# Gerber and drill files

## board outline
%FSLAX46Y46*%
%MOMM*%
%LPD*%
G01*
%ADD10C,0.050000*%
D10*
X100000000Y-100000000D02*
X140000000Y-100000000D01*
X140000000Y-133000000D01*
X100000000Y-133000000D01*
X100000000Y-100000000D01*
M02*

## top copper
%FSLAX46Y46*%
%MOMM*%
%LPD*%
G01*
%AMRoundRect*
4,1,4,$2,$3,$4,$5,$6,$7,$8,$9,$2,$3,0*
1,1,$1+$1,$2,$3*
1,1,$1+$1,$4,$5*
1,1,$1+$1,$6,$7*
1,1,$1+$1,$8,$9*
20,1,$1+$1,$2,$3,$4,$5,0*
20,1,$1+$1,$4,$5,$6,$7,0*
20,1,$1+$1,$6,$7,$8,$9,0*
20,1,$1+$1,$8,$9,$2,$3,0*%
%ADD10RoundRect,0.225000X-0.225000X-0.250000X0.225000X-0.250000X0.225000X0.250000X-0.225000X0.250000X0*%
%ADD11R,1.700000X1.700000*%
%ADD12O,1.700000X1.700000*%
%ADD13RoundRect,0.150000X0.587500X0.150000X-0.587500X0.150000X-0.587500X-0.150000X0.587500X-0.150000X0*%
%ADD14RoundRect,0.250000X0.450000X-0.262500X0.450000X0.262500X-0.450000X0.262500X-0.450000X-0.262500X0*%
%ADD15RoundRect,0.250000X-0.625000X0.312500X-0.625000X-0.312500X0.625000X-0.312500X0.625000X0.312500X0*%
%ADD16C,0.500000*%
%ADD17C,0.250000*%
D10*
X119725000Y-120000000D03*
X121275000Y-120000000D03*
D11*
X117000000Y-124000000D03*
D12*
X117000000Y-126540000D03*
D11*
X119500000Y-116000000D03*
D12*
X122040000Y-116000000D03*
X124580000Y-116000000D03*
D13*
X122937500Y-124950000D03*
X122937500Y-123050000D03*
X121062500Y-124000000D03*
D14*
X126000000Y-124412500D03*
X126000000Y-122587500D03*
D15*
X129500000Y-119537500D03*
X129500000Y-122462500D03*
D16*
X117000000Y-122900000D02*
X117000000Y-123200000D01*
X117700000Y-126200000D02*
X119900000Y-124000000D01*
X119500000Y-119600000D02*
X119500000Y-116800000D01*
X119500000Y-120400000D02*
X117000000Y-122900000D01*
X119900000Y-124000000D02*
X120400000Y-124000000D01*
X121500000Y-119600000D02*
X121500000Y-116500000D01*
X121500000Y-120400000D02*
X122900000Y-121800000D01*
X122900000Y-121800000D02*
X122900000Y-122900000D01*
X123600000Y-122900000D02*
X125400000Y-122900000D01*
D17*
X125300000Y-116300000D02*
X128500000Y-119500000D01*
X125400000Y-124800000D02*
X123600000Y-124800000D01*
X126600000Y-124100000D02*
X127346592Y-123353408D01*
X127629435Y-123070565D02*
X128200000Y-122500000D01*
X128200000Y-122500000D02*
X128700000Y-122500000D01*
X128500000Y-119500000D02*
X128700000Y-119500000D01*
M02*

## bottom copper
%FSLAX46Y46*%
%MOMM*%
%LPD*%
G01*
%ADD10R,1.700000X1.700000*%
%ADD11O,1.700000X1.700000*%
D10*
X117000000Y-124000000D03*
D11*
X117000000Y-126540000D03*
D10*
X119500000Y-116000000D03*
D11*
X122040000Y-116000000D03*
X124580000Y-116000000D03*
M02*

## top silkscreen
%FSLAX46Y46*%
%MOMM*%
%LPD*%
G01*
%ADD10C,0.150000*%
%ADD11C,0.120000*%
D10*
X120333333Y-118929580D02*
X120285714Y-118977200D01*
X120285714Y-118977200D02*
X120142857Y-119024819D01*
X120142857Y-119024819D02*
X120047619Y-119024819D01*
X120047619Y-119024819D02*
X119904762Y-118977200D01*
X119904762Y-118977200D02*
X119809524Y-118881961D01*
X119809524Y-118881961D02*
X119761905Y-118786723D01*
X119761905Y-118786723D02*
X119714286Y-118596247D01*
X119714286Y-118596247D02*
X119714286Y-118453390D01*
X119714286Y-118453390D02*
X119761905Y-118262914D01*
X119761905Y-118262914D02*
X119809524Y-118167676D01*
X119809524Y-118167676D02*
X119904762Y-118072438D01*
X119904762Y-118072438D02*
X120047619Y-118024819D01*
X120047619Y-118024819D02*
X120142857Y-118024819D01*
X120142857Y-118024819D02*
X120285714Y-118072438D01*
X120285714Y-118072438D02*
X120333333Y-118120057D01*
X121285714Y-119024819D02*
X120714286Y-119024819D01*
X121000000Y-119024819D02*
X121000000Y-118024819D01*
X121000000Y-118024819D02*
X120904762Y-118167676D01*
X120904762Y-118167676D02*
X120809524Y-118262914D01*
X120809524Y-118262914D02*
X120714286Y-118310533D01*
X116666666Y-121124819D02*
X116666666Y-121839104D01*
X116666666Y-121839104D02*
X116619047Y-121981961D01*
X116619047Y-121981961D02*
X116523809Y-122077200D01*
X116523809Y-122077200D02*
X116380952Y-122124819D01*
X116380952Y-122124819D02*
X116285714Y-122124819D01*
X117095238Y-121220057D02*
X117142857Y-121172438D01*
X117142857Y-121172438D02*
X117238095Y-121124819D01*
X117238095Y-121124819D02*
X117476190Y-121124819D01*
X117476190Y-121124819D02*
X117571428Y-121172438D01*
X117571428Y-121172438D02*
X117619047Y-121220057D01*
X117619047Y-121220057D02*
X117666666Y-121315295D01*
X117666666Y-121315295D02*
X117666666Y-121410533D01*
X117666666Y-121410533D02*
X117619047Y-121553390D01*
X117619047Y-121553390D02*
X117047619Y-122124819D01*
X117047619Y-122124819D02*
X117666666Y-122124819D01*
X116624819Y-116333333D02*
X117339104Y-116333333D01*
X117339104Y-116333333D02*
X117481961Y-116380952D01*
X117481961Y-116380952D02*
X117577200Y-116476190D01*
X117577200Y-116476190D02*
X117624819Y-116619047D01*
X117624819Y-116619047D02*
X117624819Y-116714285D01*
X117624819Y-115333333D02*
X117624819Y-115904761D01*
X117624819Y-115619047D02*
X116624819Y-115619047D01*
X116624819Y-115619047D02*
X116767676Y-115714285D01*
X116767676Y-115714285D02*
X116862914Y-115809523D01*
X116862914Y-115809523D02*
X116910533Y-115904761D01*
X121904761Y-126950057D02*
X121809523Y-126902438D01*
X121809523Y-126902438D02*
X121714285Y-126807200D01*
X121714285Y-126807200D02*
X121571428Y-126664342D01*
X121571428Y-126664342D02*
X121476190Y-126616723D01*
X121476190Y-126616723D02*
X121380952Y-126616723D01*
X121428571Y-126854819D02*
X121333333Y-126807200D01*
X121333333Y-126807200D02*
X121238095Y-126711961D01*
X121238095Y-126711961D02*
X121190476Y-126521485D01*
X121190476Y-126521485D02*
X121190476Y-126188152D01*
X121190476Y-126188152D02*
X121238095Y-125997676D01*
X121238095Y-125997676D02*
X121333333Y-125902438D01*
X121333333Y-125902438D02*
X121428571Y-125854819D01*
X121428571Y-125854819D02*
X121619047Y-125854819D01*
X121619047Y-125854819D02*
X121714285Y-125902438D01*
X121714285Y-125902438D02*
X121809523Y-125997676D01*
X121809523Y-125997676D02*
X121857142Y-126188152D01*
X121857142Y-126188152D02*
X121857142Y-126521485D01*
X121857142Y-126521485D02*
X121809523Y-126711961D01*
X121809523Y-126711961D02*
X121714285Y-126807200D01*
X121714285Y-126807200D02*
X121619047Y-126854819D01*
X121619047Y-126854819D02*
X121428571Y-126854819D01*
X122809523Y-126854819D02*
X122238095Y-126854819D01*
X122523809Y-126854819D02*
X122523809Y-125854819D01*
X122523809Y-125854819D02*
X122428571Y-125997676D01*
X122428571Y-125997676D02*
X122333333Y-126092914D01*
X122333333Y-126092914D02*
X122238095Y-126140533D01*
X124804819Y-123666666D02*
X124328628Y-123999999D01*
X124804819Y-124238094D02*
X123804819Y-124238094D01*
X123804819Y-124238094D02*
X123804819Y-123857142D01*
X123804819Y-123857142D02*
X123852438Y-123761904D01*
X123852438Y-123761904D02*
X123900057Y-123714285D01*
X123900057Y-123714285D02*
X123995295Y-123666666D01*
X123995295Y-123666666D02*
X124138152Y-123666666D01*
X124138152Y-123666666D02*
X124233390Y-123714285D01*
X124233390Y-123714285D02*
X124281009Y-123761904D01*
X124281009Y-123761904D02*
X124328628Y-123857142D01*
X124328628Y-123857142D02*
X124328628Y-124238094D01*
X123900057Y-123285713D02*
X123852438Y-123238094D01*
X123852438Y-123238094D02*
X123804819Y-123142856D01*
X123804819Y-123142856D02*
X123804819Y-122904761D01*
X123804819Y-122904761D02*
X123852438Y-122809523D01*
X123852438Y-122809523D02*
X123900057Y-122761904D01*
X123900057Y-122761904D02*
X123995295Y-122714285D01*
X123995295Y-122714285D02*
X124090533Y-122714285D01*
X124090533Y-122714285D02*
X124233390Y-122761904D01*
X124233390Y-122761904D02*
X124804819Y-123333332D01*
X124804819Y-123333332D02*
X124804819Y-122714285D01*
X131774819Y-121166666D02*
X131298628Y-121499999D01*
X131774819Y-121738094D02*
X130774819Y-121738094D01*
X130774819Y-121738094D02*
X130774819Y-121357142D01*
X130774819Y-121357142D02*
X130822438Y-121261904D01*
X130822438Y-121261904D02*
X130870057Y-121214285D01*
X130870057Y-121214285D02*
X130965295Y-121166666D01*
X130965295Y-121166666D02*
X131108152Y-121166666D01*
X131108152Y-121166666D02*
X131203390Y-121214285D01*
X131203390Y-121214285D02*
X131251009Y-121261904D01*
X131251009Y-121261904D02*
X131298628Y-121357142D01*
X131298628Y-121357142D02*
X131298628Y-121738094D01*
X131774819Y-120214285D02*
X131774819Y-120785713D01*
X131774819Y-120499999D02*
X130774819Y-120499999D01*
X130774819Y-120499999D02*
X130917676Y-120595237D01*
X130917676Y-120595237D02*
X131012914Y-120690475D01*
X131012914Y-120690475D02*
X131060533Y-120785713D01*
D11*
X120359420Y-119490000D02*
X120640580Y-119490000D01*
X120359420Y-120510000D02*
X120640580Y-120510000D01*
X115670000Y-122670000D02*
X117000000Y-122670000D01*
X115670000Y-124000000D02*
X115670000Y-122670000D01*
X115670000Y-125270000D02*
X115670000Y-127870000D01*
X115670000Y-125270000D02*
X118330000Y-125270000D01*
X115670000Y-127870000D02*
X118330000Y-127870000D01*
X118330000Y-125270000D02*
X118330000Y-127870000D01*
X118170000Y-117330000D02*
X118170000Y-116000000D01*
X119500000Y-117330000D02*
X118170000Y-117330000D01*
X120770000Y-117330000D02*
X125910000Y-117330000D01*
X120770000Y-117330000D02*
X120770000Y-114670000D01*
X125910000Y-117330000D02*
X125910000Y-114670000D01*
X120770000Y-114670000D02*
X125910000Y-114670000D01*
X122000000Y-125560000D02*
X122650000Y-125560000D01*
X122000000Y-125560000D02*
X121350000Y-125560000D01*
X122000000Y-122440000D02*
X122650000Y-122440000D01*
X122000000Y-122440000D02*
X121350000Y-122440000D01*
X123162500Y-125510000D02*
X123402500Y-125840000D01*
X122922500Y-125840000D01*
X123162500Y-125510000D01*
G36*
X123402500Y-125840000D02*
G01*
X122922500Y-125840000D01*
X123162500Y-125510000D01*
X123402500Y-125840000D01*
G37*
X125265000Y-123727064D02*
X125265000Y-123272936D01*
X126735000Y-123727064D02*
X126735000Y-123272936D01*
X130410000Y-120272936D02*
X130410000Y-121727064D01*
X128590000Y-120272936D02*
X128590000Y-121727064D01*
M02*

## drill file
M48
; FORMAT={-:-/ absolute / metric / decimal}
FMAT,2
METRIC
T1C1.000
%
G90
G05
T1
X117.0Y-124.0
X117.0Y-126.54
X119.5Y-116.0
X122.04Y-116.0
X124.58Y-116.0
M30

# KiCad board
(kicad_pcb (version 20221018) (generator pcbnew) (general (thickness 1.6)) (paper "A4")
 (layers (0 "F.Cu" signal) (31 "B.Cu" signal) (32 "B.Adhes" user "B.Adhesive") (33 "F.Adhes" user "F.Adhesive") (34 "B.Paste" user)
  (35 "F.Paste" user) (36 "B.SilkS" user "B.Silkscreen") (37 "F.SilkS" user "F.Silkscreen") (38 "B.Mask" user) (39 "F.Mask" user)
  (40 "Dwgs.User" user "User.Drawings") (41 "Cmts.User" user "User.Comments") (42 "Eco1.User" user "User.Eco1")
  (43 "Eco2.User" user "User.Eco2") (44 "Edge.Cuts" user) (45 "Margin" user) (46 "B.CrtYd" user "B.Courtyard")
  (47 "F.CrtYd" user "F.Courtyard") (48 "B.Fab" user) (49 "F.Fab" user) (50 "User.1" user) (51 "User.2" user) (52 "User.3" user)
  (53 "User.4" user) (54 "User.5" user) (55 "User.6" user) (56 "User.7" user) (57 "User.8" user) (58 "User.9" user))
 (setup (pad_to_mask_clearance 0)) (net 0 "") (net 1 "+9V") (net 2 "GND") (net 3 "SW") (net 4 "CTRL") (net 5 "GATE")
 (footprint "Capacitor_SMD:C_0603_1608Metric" (layer "F.Cu") (at 120.5 120)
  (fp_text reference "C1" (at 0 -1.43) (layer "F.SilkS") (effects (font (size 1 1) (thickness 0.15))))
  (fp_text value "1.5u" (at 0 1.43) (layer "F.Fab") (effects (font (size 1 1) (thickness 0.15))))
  (fp_line (start -0.14058 -0.51) (end 0.14058 -0.51) (stroke (width 0.12) (type solid)) (layer "F.SilkS"))
  (fp_line (start -0.14058 0.51) (end 0.14058 0.51) (stroke (width 0.12) (type solid)) (layer "F.SilkS"))
  (pad "1" smd roundrect (at -0.775 0) (size 0.9 0.95) (layers "F.Cu" "F.Paste" "F.Mask") (roundrect_rratio 0.25) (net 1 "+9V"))
  (pad "2" smd roundrect (at 0.775 0) (size 0.9 0.95) (layers "F.Cu" "F.Paste" "F.Mask") (roundrect_rratio 0.25) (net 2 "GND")))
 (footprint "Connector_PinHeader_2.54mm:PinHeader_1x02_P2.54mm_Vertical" (layer "F.Cu") (at 117 124)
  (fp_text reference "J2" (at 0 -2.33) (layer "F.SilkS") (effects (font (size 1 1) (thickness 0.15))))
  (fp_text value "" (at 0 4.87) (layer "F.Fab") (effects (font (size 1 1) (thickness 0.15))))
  (fp_line (start -1.33 -1.33) (end 0 -1.33) (stroke (width 0.12) (type solid)) (layer "F.SilkS"))
  (fp_line (start -1.33 0) (end -1.33 -1.33) (stroke (width 0.12) (type solid)) (layer "F.SilkS"))
  (fp_line (start -1.33 1.27) (end -1.33 3.87) (stroke (width 0.12) (type solid)) (layer "F.SilkS"))
  (fp_line (start -1.33 1.27) (end 1.33 1.27) (stroke (width 0.12) (type solid)) (layer "F.SilkS"))
  (fp_line (start -1.33 3.87) (end 1.33 3.87) (stroke (width 0.12) (type solid)) (layer "F.SilkS"))
  (fp_line (start 1.33 1.27) (end 1.33 3.87) (stroke (width 0.12) (type solid)) (layer "F.SilkS"))
  (pad "1" thru_hole rect (at 0 0) (size 1.7 1.7) (drill 1) (layers "*.Cu" "*.Mask") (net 1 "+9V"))
  (pad "2" thru_hole oval (at 0 2.54) (size 1.7 1.7) (drill 1) (layers "*.Cu" "*.Mask") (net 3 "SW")))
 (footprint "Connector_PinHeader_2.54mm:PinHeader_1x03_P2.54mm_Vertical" (layer "F.Cu") (at 119.5 116 90)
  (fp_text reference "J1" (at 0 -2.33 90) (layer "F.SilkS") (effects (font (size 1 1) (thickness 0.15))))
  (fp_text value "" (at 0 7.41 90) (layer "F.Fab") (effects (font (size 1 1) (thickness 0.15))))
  (fp_line (start -1.33 -1.33) (end 0 -1.33) (stroke (width 0.12) (type solid)) (layer "F.SilkS"))
  (fp_line (start -1.33 0) (end -1.33 -1.33) (stroke (width 0.12) (type solid)) (layer "F.SilkS"))
  (fp_line (start -1.33 1.27) (end -1.33 6.41) (stroke (width 0.12) (type solid)) (layer "F.SilkS"))
  (fp_line (start -1.33 1.27) (end 1.33 1.27) (stroke (width 0.12) (type solid)) (layer "F.SilkS"))
  (fp_line (start -1.33 6.41) (end 1.33 6.41) (stroke (width 0.12) (type solid)) (layer "F.SilkS"))
  (fp_line (start 1.33 1.27) (end 1.33 6.41) (stroke (width 0.12) (type solid)) (layer "F.SilkS"))
  (pad "1" thru_hole rect (at 0 0 90) (size 1.7 1.7) (drill 1) (layers "*.Cu" "*.Mask") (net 1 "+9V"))
  (pad "2" thru_hole oval (at 0 2.54 90) (size 1.7 1.7) (drill 1) (layers "*.Cu" "*.Mask") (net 2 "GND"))
  (pad "3" thru_hole oval (at 0 5.08 90) (size 1.7 1.7) (drill 1) (layers "*.Cu" "*.Mask") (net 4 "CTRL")))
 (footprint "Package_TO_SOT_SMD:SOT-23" (layer "F.Cu") (at 122 124 180)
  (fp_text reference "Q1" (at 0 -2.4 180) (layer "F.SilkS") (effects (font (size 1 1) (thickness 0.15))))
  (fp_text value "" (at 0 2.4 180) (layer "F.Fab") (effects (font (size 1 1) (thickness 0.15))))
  (fp_line (start 0 -1.56) (end -0.65 -1.56) (stroke (width 0.12) (type solid)) (layer "F.SilkS"))
  (fp_line (start 0 -1.56) (end 0.65 -1.56) (stroke (width 0.12) (type solid)) (layer "F.SilkS"))
  (fp_line (start 0 1.56) (end -0.65 1.56) (stroke (width 0.12) (type solid)) (layer "F.SilkS"))
  (fp_line (start 0 1.56) (end 0.65 1.56) (stroke (width 0.12) (type solid)) (layer "F.SilkS"))
  (fp_poly
   (pts (xy -1.1625 -1.51) (xy -1.4025 -1.84) (xy -0.9225 -1.84) (xy -1.1625 -1.51)) (stroke (width 0.12) (type solid)) (fill solid)
   (layer "F.SilkS"))
  (pad "1" smd roundrect (at -0.9375 -0.95 180) (size 1.475 0.6) (layers "F.Cu" "F.Paste" "F.Mask") (roundrect_rratio 0.25) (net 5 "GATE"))
  (pad "2" smd roundrect (at -0.9375 0.95 180) (size 1.475 0.6) (layers "F.Cu" "F.Paste" "F.Mask") (roundrect_rratio 0.25) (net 2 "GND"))
  (pad "3" smd roundrect (at 0.9375 0 180) (size 1.475 0.6) (layers "F.Cu" "F.Paste" "F.Mask") (roundrect_rratio 0.25) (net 3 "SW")))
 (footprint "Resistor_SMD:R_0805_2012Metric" (layer "F.Cu") (at 126 123.5 90)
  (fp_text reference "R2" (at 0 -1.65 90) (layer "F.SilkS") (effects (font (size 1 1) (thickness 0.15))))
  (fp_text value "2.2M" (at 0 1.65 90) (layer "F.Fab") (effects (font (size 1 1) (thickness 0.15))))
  (fp_line (start -0.227064 -0.735) (end 0.227064 -0.735) (stroke (width 0.12) (type solid)) (layer "F.SilkS"))
  (fp_line (start -0.227064 0.735) (end 0.227064 0.735) (stroke (width 0.12) (type solid)) (layer "F.SilkS"))
  (pad "1" smd roundrect (at -0.9125 0 90) (size 1.025 1.4) (layers "F.Cu" "F.Paste" "F.Mask") (roundrect_rratio 0.243902) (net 5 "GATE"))
  (pad "2" smd roundrect (at 0.9125 0 90) (size 1.025 1.4) (layers "F.Cu" "F.Paste" "F.Mask") (roundrect_rratio 0.243902) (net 2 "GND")))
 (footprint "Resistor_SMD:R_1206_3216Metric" (layer "F.Cu") (at 129.5 121 -90)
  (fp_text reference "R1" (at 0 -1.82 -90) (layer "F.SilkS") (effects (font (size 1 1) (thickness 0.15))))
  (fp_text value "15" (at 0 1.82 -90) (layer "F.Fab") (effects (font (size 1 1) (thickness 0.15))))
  (fp_line (start -0.727064 -0.91) (end 0.727064 -0.91) (stroke (width 0.12) (type solid)) (layer "F.SilkS"))
  (fp_line (start -0.727064 0.91) (end 0.727064 0.91) (stroke (width 0.12) (type solid)) (layer "F.SilkS"))
  (pad "1" smd roundrect (at -1.4625 0 270) (size 1.125 1.75) (layers "F.Cu" "F.Paste" "F.Mask") (roundrect_rratio 0.222222) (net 4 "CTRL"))
  (pad "2" smd roundrect (at 1.4625 0 270) (size 1.125 1.75) (layers "F.Cu" "F.Paste" "F.Mask") (roundrect_rratio 0.222222) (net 5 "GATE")))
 (gr_rect (start 100 100) (end 140 133) (stroke (width 0.05) (type default)) (fill none) (layer "Edge.Cuts"))
 (segment (start 117 122.9) (end 117 123.2) (width 0.5) (layer "F.Cu") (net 1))
 (segment (start 117.7 126.2) (end 119.9 124) (width 0.5) (layer "F.Cu") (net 3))
 (segment (start 119.5 119.6) (end 119.5 116.8) (width 0.5) (layer "F.Cu") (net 1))
 (segment (start 119.5 120.4) (end 117 122.9) (width 0.5) (layer "F.Cu") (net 1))
 (segment (start 119.9 124) (end 120.4 124) (width 0.5) (layer "F.Cu") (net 3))
 (segment (start 121.5 119.6) (end 121.5 116.5) (width 0.5) (layer "F.Cu") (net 2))
 (segment (start 121.5 120.4) (end 122.9 121.8) (width 0.5) (layer "F.Cu") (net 2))
 (segment (start 122.9 121.8) (end 122.9 122.9) (width 0.5) (layer "F.Cu") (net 2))
 (segment (start 123.6 122.9) (end 125.4 122.9) (width 0.5) (layer "F.Cu") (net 2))
 (segment (start 125.3 116.3) (end 128.5 119.5) (width 0.25) (layer "F.Cu") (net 4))
 (segment (start 125.4 124.8) (end 123.6 124.8) (width 0.25) (layer "F.Cu") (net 5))
 (segment (start 126.6 124.1) (end 127.346592 123.353408) (width 0.25) (layer "F.Cu") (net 5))
 (segment (start 127.629435 123.070565) (end 128.2 122.5) (width 0.25) (layer "F.Cu") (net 5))
 (segment (start 128.2 122.5) (end 128.7 122.5) (width 0.25) (layer "F.Cu") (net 5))
 (segment (start 128.5 119.5) (end 128.7 119.5) (width 0.25) (layer "F.Cu") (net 4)))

